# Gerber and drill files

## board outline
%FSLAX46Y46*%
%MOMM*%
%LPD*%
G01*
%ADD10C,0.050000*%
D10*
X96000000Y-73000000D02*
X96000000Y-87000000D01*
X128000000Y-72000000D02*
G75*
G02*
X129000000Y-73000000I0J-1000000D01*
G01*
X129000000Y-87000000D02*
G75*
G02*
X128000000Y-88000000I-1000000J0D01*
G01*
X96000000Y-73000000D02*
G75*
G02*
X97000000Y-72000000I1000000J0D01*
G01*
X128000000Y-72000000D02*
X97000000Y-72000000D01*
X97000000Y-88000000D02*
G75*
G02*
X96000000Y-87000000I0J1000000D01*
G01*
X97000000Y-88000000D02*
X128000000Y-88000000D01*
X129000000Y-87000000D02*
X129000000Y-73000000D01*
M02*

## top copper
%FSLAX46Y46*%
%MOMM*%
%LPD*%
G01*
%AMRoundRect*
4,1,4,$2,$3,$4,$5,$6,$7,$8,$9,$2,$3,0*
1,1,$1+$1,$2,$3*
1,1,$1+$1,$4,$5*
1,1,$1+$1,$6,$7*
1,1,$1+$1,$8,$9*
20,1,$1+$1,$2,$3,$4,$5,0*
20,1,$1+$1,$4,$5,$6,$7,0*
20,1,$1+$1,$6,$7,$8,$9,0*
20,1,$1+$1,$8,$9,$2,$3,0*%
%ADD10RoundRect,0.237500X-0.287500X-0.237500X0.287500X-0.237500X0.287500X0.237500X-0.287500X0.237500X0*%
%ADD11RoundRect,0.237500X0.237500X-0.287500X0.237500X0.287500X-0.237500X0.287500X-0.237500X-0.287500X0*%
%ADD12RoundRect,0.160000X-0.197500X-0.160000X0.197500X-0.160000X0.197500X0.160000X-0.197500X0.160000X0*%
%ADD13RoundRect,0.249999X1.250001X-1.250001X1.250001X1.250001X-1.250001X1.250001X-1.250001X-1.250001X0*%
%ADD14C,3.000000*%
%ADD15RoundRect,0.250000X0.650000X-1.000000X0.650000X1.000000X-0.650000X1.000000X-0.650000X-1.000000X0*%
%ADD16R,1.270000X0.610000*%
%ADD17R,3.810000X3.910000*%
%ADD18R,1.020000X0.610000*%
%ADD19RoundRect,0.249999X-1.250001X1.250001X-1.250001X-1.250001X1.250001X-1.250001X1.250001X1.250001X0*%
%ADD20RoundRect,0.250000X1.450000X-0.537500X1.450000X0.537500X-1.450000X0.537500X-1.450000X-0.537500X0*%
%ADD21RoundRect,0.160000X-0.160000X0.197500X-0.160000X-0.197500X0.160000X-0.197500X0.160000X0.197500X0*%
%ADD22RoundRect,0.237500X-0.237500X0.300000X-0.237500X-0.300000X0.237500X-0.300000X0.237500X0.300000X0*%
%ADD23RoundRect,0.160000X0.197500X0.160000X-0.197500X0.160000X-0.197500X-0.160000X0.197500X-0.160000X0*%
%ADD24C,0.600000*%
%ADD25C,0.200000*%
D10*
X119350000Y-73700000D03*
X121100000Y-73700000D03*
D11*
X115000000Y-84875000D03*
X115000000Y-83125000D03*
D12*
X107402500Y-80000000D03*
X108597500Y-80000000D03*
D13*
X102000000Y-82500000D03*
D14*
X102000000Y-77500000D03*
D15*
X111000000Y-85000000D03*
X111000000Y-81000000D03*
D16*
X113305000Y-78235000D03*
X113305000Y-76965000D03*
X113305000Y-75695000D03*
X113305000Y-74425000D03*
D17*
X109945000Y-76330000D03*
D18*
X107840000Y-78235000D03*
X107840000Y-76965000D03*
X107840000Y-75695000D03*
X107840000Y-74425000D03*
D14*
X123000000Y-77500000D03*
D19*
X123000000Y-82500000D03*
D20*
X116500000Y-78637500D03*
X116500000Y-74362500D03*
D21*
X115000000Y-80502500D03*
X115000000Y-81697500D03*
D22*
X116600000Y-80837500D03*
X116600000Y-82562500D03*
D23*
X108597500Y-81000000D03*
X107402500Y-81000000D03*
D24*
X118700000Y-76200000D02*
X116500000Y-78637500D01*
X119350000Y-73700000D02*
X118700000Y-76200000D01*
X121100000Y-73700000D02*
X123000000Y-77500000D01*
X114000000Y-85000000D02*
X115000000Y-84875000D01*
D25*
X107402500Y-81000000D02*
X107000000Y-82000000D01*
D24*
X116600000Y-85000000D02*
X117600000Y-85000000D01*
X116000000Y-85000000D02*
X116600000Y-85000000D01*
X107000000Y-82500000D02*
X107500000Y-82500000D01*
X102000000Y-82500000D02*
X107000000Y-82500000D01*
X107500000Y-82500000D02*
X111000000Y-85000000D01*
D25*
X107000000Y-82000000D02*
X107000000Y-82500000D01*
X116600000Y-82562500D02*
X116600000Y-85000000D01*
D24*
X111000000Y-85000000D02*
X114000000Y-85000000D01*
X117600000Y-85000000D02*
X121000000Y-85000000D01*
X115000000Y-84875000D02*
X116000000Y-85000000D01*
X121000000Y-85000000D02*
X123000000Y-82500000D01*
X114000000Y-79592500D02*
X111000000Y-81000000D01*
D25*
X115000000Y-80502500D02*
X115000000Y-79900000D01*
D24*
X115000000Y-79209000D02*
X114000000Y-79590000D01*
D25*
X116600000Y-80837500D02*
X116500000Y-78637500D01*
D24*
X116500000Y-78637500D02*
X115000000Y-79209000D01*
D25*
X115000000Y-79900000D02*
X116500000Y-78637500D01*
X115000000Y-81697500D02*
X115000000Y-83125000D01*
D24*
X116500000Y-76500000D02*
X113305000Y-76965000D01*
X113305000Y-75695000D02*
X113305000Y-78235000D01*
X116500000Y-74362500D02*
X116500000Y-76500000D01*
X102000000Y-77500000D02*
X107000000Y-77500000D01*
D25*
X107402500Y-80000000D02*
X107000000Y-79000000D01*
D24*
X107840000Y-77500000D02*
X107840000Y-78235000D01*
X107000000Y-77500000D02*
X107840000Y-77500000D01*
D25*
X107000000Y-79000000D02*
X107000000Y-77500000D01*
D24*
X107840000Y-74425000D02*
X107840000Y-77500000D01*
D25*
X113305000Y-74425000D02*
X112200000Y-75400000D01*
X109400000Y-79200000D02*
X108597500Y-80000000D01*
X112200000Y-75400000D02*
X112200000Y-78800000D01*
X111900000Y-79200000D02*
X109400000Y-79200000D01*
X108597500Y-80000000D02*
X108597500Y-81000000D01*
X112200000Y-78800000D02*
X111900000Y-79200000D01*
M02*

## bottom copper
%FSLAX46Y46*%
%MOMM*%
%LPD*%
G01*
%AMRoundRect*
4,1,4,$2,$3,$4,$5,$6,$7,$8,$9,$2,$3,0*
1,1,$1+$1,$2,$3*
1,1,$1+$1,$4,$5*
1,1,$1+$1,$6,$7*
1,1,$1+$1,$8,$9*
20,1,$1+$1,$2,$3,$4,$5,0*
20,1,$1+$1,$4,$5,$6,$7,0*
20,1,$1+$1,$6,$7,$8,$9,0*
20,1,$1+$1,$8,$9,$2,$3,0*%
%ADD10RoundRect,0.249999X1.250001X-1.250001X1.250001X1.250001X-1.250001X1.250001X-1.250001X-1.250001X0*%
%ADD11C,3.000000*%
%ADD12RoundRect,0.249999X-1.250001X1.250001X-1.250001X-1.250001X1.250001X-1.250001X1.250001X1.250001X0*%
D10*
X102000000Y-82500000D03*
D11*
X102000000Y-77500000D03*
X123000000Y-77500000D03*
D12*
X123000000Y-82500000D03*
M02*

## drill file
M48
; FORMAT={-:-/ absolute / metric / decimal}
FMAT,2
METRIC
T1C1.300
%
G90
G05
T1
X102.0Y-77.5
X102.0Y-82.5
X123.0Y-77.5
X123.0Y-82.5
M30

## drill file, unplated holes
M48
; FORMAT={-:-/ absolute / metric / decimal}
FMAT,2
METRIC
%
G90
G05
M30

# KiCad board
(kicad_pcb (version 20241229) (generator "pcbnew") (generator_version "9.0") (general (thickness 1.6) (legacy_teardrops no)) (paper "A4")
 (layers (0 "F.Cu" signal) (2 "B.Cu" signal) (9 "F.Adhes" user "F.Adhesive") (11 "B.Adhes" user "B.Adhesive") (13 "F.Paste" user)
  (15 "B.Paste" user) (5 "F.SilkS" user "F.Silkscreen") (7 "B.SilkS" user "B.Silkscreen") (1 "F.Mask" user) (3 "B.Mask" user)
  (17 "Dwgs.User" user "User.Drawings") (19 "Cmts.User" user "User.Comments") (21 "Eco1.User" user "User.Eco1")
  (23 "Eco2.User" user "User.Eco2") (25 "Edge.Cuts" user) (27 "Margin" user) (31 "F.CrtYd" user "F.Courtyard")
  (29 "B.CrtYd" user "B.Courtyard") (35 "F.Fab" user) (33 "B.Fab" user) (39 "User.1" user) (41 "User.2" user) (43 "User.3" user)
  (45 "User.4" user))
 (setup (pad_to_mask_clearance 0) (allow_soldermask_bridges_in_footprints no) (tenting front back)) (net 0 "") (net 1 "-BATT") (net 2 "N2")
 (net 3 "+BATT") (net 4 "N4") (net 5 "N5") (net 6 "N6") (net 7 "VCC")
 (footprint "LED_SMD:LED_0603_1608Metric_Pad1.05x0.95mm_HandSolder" (layer "F.Cu") (at 115 84 90)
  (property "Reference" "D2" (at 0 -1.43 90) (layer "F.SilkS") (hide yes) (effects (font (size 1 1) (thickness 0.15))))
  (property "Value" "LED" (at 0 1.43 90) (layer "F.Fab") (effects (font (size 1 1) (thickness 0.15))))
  (pad "1" smd roundrect (at -0.875 0 90) (size 1.05 0.95) (layers "F.Cu" "F.Mask" "F.Paste") (roundrect_rratio 0.25) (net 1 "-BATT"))
  (pad "2" smd roundrect (at 0.875 0 90) (size 1.05 0.95) (layers "F.Cu" "F.Mask" "F.Paste") (roundrect_rratio 0.25) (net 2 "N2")))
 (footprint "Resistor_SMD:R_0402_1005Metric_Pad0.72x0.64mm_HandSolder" (layer "F.Cu") (at 108 80)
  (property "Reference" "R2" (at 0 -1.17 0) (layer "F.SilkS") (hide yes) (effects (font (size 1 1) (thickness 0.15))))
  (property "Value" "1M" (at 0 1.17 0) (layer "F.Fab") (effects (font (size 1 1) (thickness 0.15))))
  (pad "1" smd roundrect (at -0.5975 0) (size 0.715 0.64) (layers "F.Cu" "F.Mask" "F.Paste") (roundrect_rratio 0.25) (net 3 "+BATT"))
  (pad "2" smd roundrect (at 0.5975 0) (size 0.715 0.64) (layers "F.Cu" "F.Mask" "F.Paste") (roundrect_rratio 0.25) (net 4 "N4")))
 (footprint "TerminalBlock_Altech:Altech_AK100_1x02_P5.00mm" (layer "F.Cu") (at 102 82.5 90)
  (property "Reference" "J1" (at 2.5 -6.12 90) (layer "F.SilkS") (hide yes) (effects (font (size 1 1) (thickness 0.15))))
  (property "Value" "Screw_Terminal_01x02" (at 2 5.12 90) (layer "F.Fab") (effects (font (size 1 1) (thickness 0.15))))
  (pad "1" thru_hole roundrect (at 0 0 90) (size 3 3) (drill 1.3) (layers "*.Cu" "*.Mask") (remove_unused_layers no)
   (roundrect_rratio 0.083333) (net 1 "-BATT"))
  (pad "2" thru_hole circle (at 5 0 90) (size 3 3) (drill 1.3) (layers "*.Cu" "*.Mask") (remove_unused_layers no) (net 3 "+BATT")))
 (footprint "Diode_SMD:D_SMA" (layer "F.Cu") (at 111 83 90)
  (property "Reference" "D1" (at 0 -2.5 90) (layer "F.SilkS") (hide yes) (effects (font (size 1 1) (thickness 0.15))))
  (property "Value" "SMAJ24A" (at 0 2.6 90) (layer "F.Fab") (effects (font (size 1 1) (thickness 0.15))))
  (pad "1" smd roundrect (at -2 0 90) (size 2.5 1.8) (layers "F.Cu" "F.Mask" "F.Paste") (roundrect_rratio 0.1388888889) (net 1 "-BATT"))
  (pad "2" smd roundrect (at 2 0 90) (size 2.5 1.8) (layers "F.Cu" "F.Mask" "F.Paste") (roundrect_rratio 0.1388888889) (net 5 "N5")))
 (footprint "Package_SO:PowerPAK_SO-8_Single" (layer "F.Cu") (at 110.635 76.33 180)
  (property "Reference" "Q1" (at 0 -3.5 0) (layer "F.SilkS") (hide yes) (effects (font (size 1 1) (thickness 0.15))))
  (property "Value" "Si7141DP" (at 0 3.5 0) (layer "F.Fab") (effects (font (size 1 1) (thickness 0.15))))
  (pad "1" smd rect (at -2.67 -1.905 180) (size 1.27 0.61) (layers "F.Cu" "F.Mask" "F.Paste") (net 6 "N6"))
  (pad "2" smd rect (at -2.67 -0.635 180) (size 1.27 0.61) (layers "F.Cu" "F.Mask" "F.Paste") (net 6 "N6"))
  (pad "3" smd rect (at -2.67 0.635 180) (size 1.27 0.61) (layers "F.Cu" "F.Mask" "F.Paste") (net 6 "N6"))
  (pad "4" smd rect (at -2.67 1.905 180) (size 1.27 0.61) (layers "F.Cu" "F.Mask" "F.Paste") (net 4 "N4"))
  (pad "5" smd rect (at 0.69 0 180) (size 3.81 3.91) (layers "F.Cu" "F.Mask" "F.Paste") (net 3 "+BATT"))
  (pad "5" smd rect (at 2.795 -1.905 180) (size 1.02 0.61) (layers "F.Cu" "F.Mask" "F.Paste") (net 3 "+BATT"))
  (pad "5" smd rect (at 2.795 -0.635 180) (size 1.02 0.61) (layers "F.Cu" "F.Mask" "F.Paste") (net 3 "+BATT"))
  (pad "5" smd rect (at 2.795 0.635 180) (size 1.02 0.61) (layers "F.Cu" "F.Mask" "F.Paste") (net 3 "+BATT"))
  (pad "5" smd rect (at 2.795 1.905 180) (size 1.02 0.61) (layers "F.Cu" "F.Mask" "F.Paste") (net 3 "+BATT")))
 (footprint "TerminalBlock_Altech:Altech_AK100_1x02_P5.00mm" (layer "F.Cu") (at 123 77.5 -90)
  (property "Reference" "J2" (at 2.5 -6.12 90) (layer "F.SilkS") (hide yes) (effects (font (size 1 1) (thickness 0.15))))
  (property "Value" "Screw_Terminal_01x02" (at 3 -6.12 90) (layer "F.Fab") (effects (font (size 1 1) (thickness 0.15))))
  (pad "1" thru_hole circle (at 0 0 270) (size 3 3) (drill 1.3) (layers "*.Cu" "*.Mask") (remove_unused_layers no) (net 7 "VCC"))
  (pad "2" thru_hole roundrect (at 5 0 270) (size 3 3) (drill 1.3) (layers "*.Cu" "*.Mask") (remove_unused_layers no)
   (roundrect_rratio 0.083333) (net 1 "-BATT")))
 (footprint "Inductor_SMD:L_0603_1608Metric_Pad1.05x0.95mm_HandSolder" (layer "F.Cu") (at 120.225 73.7)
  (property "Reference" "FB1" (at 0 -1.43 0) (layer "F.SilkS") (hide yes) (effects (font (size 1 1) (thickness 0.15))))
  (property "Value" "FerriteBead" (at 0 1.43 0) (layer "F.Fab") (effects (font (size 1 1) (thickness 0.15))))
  (pad "1" smd roundrect (at -0.875 0) (size 1.05 0.95) (layers "F.Cu" "F.Mask" "F.Paste") (roundrect_rratio 0.25) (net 5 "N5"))
  (pad "2" smd roundrect (at 0.875 0) (size 1.05 0.95) (layers "F.Cu" "F.Mask" "F.Paste") (roundrect_rratio 0.25) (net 7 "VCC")))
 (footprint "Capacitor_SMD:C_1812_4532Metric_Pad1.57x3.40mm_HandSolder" (layer "F.Cu") (at 116.5 76.5 90)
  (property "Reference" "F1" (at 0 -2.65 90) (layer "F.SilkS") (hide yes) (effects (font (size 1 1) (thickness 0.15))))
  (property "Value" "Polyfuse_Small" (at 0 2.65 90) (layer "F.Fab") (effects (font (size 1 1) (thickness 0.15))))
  (pad "1" smd roundrect (at -2.1375 0 90) (size 1.575 3.4) (layers "F.Cu" "F.Mask" "F.Paste") (roundrect_rratio 0.15873) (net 5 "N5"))
  (pad "2" smd roundrect (at 2.1375 0 90) (size 1.575 3.4) (layers "F.Cu" "F.Mask" "F.Paste") (roundrect_rratio 0.15873) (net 6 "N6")))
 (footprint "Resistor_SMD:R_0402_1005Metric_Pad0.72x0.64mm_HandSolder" (layer "F.Cu") (at 115 81.1 -90)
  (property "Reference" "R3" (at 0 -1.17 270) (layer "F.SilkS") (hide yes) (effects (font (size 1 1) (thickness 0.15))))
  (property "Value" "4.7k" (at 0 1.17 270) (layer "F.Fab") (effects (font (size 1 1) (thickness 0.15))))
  (pad "1" smd roundrect (at -0.5975 0 270) (size 0.715 0.64) (layers "F.Cu" "F.Mask" "F.Paste") (roundrect_rratio 0.25) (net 5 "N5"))
  (pad "2" smd roundrect (at 0.5975 0 270) (size 0.715 0.64) (layers "F.Cu" "F.Mask" "F.Paste") (roundrect_rratio 0.25) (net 2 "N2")))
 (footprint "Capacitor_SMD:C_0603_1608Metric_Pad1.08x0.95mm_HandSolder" (layer "F.Cu") (at 116.6 81.7 -90)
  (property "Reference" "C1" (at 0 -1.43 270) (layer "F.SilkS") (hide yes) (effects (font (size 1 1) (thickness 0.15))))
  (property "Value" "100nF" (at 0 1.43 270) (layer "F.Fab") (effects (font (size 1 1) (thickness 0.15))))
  (pad "1" smd roundrect (at -0.8625 0 270) (size 1.075 0.95) (layers "F.Cu" "F.Mask" "F.Paste") (roundrect_rratio 0.25) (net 5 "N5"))
  (pad "2" smd roundrect (at 0.8625 0 270) (size 1.075 0.95) (layers "F.Cu" "F.Mask" "F.Paste") (roundrect_rratio 0.25) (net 1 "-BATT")))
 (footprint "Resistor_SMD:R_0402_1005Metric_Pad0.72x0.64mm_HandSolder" (layer "F.Cu") (at 108 81 180)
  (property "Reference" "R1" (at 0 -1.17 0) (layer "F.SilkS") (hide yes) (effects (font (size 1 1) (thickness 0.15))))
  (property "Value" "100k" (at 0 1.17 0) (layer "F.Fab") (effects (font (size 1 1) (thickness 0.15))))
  (pad "1" smd roundrect (at -0.5975 0 180) (size 0.715 0.64) (layers "F.Cu" "F.Mask" "F.Paste") (roundrect_rratio 0.25) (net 4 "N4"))
  (pad "2" smd roundrect (at 0.5975 0 180) (size 0.715 0.64) (layers "F.Cu" "F.Mask" "F.Paste") (roundrect_rratio 0.25) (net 1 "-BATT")))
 (gr_line (start 96 73) (end 96 87) (stroke (width 0.05) (type default)) (layer "Edge.Cuts"))
 (gr_arc (start 128 72) (mid 128.707107 72.292893) (end 129 73) (stroke (width 0.05) (type default)) (layer "Edge.Cuts"))
 (gr_arc (start 129 87) (mid 128.707107 87.707107) (end 128 88) (stroke (width 0.05) (type default)) (layer "Edge.Cuts"))
 (gr_arc (start 96 73) (mid 96.292893 72.292893) (end 97 72) (stroke (width 0.05) (type default)) (layer "Edge.Cuts"))
 (gr_line (start 128 72) (end 97 72) (stroke (width 0.05) (type default)) (layer "Edge.Cuts"))
 (gr_arc (start 97 88) (mid 96.292893 87.707107) (end 96 87) (stroke (width 0.05) (type default)) (layer "Edge.Cuts"))
 (gr_line (start 97 88) (end 128 88) (stroke (width 0.05) (type default)) (layer "Edge.Cuts"))
 (gr_line (start 129 87) (end 129 73) (stroke (width 0.05) (type default)) (layer "Edge.Cuts"))
 (segment (start 114 85) (end 115 84.875) (width 0.6) (layer "F.Cu") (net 1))
 (segment (start 107.4025 81) (end 107 82) (width 0.2) (layer "F.Cu") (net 1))
 (segment (start 116.6 85) (end 117.6 85) (width 0.6) (layer "F.Cu") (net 1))
 (segment (start 116 85) (end 116.6 85) (width 0.6) (layer "F.Cu") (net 1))
 (segment (start 107 82.5) (end 107.5 82.5) (width 0.6) (layer "F.Cu") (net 1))
 (segment (start 102 82.5) (end 107 82.5) (width 0.6) (layer "F.Cu") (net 1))
 (segment (start 107.5 82.5) (end 111 85) (width 0.6) (layer "F.Cu") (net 1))
 (segment (start 107 82) (end 107 82.5) (width 0.2) (layer "F.Cu") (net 1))
 (segment (start 116.6 82.5625) (end 116.6 85) (width 0.2) (layer "F.Cu") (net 1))
 (segment (start 111 85) (end 114 85) (width 0.6) (layer "F.Cu") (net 1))
 (segment (start 117.6 85) (end 121 85) (width 0.6) (layer "F.Cu") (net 1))
 (segment (start 115 84.875) (end 116 85) (width 0.6) (layer "F.Cu") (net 1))
 (segment (start 121 85) (end 123 82.5) (width 0.6) (layer "F.Cu") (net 1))
 (segment (start 121.1 73.7) (end 123 77.5) (width 0.6) (layer "F.Cu") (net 7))
 (segment (start 115 81.6975) (end 115 83.125) (width 0.2) (layer "F.Cu") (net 2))
 (segment (start 116.5 76.5) (end 113.305 76.965) (width 0.6) (layer "F.Cu") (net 6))
 (segment (start 113.305 75.695) (end 113.305 78.235) (width 0.6) (layer "F.Cu") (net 6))
 (segment (start 116.5 74.3625) (end 116.5 76.5) (width 0.6) (layer "F.Cu") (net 6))
 (segment (start 102 77.5) (end 107 77.5) (width 0.6) (layer "F.Cu") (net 3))
 (segment (start 107.4025 80) (end 107 79) (width 0.2) (layer "F.Cu") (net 3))
 (segment (start 107.84 77.5) (end 107.84 78.235) (width 0.6) (layer "F.Cu") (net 3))
 (segment (start 107 77.5) (end 107.84 77.5) (width 0.6) (layer "F.Cu") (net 3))
 (segment (start 107 79) (end 107 77.5) (width 0.2) (layer "F.Cu") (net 3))
 (segment (start 107.84 74.425) (end 107.84 77.5) (width 0.6) (layer "F.Cu") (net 3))
 (segment (start 113.305 74.425) (end 112.2 75.4) (width 0.2) (layer "F.Cu") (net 4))
 (segment (start 109.4 79.2) (end 108.5975 80) (width 0.2) (layer "F.Cu") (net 4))
 (segment (start 112.2 75.4) (end 112.2 78.8) (width 0.2) (layer "F.Cu") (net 4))
 (segment (start 111.9 79.2) (end 109.4 79.2) (width 0.2) (layer "F.Cu") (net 4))
 (segment (start 108.5975 80) (end 108.5975 81) (width 0.2) (layer "F.Cu") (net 4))
 (segment (start 112.2 78.8) (end 111.9 79.2) (width 0.2) (layer "F.Cu") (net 4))
 (segment (start 114 79.5925) (end 111 81) (width 0.6) (layer "F.Cu") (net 5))
 (segment (start 118.7 76.2) (end 116.5 78.6375) (width 0.6) (layer "F.Cu") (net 5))
 (segment (start 115 80.5025) (end 115 79.9) (width 0.2) (layer "F.Cu") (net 5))
 (segment (start 115 79.209) (end 114 79.59) (width 0.6) (layer "F.Cu") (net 5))
 (segment (start 116.6 80.8375) (end 116.5 78.6375) (width 0.2) (layer "F.Cu") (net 5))
 (segment (start 119.35 73.7) (end 118.7 76.2) (width 0.6) (layer "F.Cu") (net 5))
 (segment (start 116.5 78.6375) (end 115 79.209) (width 0.6) (layer "F.Cu") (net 5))
 (segment (start 115 79.9) (end 116.5 78.6375) (width 0.2) (layer "F.Cu") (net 5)))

